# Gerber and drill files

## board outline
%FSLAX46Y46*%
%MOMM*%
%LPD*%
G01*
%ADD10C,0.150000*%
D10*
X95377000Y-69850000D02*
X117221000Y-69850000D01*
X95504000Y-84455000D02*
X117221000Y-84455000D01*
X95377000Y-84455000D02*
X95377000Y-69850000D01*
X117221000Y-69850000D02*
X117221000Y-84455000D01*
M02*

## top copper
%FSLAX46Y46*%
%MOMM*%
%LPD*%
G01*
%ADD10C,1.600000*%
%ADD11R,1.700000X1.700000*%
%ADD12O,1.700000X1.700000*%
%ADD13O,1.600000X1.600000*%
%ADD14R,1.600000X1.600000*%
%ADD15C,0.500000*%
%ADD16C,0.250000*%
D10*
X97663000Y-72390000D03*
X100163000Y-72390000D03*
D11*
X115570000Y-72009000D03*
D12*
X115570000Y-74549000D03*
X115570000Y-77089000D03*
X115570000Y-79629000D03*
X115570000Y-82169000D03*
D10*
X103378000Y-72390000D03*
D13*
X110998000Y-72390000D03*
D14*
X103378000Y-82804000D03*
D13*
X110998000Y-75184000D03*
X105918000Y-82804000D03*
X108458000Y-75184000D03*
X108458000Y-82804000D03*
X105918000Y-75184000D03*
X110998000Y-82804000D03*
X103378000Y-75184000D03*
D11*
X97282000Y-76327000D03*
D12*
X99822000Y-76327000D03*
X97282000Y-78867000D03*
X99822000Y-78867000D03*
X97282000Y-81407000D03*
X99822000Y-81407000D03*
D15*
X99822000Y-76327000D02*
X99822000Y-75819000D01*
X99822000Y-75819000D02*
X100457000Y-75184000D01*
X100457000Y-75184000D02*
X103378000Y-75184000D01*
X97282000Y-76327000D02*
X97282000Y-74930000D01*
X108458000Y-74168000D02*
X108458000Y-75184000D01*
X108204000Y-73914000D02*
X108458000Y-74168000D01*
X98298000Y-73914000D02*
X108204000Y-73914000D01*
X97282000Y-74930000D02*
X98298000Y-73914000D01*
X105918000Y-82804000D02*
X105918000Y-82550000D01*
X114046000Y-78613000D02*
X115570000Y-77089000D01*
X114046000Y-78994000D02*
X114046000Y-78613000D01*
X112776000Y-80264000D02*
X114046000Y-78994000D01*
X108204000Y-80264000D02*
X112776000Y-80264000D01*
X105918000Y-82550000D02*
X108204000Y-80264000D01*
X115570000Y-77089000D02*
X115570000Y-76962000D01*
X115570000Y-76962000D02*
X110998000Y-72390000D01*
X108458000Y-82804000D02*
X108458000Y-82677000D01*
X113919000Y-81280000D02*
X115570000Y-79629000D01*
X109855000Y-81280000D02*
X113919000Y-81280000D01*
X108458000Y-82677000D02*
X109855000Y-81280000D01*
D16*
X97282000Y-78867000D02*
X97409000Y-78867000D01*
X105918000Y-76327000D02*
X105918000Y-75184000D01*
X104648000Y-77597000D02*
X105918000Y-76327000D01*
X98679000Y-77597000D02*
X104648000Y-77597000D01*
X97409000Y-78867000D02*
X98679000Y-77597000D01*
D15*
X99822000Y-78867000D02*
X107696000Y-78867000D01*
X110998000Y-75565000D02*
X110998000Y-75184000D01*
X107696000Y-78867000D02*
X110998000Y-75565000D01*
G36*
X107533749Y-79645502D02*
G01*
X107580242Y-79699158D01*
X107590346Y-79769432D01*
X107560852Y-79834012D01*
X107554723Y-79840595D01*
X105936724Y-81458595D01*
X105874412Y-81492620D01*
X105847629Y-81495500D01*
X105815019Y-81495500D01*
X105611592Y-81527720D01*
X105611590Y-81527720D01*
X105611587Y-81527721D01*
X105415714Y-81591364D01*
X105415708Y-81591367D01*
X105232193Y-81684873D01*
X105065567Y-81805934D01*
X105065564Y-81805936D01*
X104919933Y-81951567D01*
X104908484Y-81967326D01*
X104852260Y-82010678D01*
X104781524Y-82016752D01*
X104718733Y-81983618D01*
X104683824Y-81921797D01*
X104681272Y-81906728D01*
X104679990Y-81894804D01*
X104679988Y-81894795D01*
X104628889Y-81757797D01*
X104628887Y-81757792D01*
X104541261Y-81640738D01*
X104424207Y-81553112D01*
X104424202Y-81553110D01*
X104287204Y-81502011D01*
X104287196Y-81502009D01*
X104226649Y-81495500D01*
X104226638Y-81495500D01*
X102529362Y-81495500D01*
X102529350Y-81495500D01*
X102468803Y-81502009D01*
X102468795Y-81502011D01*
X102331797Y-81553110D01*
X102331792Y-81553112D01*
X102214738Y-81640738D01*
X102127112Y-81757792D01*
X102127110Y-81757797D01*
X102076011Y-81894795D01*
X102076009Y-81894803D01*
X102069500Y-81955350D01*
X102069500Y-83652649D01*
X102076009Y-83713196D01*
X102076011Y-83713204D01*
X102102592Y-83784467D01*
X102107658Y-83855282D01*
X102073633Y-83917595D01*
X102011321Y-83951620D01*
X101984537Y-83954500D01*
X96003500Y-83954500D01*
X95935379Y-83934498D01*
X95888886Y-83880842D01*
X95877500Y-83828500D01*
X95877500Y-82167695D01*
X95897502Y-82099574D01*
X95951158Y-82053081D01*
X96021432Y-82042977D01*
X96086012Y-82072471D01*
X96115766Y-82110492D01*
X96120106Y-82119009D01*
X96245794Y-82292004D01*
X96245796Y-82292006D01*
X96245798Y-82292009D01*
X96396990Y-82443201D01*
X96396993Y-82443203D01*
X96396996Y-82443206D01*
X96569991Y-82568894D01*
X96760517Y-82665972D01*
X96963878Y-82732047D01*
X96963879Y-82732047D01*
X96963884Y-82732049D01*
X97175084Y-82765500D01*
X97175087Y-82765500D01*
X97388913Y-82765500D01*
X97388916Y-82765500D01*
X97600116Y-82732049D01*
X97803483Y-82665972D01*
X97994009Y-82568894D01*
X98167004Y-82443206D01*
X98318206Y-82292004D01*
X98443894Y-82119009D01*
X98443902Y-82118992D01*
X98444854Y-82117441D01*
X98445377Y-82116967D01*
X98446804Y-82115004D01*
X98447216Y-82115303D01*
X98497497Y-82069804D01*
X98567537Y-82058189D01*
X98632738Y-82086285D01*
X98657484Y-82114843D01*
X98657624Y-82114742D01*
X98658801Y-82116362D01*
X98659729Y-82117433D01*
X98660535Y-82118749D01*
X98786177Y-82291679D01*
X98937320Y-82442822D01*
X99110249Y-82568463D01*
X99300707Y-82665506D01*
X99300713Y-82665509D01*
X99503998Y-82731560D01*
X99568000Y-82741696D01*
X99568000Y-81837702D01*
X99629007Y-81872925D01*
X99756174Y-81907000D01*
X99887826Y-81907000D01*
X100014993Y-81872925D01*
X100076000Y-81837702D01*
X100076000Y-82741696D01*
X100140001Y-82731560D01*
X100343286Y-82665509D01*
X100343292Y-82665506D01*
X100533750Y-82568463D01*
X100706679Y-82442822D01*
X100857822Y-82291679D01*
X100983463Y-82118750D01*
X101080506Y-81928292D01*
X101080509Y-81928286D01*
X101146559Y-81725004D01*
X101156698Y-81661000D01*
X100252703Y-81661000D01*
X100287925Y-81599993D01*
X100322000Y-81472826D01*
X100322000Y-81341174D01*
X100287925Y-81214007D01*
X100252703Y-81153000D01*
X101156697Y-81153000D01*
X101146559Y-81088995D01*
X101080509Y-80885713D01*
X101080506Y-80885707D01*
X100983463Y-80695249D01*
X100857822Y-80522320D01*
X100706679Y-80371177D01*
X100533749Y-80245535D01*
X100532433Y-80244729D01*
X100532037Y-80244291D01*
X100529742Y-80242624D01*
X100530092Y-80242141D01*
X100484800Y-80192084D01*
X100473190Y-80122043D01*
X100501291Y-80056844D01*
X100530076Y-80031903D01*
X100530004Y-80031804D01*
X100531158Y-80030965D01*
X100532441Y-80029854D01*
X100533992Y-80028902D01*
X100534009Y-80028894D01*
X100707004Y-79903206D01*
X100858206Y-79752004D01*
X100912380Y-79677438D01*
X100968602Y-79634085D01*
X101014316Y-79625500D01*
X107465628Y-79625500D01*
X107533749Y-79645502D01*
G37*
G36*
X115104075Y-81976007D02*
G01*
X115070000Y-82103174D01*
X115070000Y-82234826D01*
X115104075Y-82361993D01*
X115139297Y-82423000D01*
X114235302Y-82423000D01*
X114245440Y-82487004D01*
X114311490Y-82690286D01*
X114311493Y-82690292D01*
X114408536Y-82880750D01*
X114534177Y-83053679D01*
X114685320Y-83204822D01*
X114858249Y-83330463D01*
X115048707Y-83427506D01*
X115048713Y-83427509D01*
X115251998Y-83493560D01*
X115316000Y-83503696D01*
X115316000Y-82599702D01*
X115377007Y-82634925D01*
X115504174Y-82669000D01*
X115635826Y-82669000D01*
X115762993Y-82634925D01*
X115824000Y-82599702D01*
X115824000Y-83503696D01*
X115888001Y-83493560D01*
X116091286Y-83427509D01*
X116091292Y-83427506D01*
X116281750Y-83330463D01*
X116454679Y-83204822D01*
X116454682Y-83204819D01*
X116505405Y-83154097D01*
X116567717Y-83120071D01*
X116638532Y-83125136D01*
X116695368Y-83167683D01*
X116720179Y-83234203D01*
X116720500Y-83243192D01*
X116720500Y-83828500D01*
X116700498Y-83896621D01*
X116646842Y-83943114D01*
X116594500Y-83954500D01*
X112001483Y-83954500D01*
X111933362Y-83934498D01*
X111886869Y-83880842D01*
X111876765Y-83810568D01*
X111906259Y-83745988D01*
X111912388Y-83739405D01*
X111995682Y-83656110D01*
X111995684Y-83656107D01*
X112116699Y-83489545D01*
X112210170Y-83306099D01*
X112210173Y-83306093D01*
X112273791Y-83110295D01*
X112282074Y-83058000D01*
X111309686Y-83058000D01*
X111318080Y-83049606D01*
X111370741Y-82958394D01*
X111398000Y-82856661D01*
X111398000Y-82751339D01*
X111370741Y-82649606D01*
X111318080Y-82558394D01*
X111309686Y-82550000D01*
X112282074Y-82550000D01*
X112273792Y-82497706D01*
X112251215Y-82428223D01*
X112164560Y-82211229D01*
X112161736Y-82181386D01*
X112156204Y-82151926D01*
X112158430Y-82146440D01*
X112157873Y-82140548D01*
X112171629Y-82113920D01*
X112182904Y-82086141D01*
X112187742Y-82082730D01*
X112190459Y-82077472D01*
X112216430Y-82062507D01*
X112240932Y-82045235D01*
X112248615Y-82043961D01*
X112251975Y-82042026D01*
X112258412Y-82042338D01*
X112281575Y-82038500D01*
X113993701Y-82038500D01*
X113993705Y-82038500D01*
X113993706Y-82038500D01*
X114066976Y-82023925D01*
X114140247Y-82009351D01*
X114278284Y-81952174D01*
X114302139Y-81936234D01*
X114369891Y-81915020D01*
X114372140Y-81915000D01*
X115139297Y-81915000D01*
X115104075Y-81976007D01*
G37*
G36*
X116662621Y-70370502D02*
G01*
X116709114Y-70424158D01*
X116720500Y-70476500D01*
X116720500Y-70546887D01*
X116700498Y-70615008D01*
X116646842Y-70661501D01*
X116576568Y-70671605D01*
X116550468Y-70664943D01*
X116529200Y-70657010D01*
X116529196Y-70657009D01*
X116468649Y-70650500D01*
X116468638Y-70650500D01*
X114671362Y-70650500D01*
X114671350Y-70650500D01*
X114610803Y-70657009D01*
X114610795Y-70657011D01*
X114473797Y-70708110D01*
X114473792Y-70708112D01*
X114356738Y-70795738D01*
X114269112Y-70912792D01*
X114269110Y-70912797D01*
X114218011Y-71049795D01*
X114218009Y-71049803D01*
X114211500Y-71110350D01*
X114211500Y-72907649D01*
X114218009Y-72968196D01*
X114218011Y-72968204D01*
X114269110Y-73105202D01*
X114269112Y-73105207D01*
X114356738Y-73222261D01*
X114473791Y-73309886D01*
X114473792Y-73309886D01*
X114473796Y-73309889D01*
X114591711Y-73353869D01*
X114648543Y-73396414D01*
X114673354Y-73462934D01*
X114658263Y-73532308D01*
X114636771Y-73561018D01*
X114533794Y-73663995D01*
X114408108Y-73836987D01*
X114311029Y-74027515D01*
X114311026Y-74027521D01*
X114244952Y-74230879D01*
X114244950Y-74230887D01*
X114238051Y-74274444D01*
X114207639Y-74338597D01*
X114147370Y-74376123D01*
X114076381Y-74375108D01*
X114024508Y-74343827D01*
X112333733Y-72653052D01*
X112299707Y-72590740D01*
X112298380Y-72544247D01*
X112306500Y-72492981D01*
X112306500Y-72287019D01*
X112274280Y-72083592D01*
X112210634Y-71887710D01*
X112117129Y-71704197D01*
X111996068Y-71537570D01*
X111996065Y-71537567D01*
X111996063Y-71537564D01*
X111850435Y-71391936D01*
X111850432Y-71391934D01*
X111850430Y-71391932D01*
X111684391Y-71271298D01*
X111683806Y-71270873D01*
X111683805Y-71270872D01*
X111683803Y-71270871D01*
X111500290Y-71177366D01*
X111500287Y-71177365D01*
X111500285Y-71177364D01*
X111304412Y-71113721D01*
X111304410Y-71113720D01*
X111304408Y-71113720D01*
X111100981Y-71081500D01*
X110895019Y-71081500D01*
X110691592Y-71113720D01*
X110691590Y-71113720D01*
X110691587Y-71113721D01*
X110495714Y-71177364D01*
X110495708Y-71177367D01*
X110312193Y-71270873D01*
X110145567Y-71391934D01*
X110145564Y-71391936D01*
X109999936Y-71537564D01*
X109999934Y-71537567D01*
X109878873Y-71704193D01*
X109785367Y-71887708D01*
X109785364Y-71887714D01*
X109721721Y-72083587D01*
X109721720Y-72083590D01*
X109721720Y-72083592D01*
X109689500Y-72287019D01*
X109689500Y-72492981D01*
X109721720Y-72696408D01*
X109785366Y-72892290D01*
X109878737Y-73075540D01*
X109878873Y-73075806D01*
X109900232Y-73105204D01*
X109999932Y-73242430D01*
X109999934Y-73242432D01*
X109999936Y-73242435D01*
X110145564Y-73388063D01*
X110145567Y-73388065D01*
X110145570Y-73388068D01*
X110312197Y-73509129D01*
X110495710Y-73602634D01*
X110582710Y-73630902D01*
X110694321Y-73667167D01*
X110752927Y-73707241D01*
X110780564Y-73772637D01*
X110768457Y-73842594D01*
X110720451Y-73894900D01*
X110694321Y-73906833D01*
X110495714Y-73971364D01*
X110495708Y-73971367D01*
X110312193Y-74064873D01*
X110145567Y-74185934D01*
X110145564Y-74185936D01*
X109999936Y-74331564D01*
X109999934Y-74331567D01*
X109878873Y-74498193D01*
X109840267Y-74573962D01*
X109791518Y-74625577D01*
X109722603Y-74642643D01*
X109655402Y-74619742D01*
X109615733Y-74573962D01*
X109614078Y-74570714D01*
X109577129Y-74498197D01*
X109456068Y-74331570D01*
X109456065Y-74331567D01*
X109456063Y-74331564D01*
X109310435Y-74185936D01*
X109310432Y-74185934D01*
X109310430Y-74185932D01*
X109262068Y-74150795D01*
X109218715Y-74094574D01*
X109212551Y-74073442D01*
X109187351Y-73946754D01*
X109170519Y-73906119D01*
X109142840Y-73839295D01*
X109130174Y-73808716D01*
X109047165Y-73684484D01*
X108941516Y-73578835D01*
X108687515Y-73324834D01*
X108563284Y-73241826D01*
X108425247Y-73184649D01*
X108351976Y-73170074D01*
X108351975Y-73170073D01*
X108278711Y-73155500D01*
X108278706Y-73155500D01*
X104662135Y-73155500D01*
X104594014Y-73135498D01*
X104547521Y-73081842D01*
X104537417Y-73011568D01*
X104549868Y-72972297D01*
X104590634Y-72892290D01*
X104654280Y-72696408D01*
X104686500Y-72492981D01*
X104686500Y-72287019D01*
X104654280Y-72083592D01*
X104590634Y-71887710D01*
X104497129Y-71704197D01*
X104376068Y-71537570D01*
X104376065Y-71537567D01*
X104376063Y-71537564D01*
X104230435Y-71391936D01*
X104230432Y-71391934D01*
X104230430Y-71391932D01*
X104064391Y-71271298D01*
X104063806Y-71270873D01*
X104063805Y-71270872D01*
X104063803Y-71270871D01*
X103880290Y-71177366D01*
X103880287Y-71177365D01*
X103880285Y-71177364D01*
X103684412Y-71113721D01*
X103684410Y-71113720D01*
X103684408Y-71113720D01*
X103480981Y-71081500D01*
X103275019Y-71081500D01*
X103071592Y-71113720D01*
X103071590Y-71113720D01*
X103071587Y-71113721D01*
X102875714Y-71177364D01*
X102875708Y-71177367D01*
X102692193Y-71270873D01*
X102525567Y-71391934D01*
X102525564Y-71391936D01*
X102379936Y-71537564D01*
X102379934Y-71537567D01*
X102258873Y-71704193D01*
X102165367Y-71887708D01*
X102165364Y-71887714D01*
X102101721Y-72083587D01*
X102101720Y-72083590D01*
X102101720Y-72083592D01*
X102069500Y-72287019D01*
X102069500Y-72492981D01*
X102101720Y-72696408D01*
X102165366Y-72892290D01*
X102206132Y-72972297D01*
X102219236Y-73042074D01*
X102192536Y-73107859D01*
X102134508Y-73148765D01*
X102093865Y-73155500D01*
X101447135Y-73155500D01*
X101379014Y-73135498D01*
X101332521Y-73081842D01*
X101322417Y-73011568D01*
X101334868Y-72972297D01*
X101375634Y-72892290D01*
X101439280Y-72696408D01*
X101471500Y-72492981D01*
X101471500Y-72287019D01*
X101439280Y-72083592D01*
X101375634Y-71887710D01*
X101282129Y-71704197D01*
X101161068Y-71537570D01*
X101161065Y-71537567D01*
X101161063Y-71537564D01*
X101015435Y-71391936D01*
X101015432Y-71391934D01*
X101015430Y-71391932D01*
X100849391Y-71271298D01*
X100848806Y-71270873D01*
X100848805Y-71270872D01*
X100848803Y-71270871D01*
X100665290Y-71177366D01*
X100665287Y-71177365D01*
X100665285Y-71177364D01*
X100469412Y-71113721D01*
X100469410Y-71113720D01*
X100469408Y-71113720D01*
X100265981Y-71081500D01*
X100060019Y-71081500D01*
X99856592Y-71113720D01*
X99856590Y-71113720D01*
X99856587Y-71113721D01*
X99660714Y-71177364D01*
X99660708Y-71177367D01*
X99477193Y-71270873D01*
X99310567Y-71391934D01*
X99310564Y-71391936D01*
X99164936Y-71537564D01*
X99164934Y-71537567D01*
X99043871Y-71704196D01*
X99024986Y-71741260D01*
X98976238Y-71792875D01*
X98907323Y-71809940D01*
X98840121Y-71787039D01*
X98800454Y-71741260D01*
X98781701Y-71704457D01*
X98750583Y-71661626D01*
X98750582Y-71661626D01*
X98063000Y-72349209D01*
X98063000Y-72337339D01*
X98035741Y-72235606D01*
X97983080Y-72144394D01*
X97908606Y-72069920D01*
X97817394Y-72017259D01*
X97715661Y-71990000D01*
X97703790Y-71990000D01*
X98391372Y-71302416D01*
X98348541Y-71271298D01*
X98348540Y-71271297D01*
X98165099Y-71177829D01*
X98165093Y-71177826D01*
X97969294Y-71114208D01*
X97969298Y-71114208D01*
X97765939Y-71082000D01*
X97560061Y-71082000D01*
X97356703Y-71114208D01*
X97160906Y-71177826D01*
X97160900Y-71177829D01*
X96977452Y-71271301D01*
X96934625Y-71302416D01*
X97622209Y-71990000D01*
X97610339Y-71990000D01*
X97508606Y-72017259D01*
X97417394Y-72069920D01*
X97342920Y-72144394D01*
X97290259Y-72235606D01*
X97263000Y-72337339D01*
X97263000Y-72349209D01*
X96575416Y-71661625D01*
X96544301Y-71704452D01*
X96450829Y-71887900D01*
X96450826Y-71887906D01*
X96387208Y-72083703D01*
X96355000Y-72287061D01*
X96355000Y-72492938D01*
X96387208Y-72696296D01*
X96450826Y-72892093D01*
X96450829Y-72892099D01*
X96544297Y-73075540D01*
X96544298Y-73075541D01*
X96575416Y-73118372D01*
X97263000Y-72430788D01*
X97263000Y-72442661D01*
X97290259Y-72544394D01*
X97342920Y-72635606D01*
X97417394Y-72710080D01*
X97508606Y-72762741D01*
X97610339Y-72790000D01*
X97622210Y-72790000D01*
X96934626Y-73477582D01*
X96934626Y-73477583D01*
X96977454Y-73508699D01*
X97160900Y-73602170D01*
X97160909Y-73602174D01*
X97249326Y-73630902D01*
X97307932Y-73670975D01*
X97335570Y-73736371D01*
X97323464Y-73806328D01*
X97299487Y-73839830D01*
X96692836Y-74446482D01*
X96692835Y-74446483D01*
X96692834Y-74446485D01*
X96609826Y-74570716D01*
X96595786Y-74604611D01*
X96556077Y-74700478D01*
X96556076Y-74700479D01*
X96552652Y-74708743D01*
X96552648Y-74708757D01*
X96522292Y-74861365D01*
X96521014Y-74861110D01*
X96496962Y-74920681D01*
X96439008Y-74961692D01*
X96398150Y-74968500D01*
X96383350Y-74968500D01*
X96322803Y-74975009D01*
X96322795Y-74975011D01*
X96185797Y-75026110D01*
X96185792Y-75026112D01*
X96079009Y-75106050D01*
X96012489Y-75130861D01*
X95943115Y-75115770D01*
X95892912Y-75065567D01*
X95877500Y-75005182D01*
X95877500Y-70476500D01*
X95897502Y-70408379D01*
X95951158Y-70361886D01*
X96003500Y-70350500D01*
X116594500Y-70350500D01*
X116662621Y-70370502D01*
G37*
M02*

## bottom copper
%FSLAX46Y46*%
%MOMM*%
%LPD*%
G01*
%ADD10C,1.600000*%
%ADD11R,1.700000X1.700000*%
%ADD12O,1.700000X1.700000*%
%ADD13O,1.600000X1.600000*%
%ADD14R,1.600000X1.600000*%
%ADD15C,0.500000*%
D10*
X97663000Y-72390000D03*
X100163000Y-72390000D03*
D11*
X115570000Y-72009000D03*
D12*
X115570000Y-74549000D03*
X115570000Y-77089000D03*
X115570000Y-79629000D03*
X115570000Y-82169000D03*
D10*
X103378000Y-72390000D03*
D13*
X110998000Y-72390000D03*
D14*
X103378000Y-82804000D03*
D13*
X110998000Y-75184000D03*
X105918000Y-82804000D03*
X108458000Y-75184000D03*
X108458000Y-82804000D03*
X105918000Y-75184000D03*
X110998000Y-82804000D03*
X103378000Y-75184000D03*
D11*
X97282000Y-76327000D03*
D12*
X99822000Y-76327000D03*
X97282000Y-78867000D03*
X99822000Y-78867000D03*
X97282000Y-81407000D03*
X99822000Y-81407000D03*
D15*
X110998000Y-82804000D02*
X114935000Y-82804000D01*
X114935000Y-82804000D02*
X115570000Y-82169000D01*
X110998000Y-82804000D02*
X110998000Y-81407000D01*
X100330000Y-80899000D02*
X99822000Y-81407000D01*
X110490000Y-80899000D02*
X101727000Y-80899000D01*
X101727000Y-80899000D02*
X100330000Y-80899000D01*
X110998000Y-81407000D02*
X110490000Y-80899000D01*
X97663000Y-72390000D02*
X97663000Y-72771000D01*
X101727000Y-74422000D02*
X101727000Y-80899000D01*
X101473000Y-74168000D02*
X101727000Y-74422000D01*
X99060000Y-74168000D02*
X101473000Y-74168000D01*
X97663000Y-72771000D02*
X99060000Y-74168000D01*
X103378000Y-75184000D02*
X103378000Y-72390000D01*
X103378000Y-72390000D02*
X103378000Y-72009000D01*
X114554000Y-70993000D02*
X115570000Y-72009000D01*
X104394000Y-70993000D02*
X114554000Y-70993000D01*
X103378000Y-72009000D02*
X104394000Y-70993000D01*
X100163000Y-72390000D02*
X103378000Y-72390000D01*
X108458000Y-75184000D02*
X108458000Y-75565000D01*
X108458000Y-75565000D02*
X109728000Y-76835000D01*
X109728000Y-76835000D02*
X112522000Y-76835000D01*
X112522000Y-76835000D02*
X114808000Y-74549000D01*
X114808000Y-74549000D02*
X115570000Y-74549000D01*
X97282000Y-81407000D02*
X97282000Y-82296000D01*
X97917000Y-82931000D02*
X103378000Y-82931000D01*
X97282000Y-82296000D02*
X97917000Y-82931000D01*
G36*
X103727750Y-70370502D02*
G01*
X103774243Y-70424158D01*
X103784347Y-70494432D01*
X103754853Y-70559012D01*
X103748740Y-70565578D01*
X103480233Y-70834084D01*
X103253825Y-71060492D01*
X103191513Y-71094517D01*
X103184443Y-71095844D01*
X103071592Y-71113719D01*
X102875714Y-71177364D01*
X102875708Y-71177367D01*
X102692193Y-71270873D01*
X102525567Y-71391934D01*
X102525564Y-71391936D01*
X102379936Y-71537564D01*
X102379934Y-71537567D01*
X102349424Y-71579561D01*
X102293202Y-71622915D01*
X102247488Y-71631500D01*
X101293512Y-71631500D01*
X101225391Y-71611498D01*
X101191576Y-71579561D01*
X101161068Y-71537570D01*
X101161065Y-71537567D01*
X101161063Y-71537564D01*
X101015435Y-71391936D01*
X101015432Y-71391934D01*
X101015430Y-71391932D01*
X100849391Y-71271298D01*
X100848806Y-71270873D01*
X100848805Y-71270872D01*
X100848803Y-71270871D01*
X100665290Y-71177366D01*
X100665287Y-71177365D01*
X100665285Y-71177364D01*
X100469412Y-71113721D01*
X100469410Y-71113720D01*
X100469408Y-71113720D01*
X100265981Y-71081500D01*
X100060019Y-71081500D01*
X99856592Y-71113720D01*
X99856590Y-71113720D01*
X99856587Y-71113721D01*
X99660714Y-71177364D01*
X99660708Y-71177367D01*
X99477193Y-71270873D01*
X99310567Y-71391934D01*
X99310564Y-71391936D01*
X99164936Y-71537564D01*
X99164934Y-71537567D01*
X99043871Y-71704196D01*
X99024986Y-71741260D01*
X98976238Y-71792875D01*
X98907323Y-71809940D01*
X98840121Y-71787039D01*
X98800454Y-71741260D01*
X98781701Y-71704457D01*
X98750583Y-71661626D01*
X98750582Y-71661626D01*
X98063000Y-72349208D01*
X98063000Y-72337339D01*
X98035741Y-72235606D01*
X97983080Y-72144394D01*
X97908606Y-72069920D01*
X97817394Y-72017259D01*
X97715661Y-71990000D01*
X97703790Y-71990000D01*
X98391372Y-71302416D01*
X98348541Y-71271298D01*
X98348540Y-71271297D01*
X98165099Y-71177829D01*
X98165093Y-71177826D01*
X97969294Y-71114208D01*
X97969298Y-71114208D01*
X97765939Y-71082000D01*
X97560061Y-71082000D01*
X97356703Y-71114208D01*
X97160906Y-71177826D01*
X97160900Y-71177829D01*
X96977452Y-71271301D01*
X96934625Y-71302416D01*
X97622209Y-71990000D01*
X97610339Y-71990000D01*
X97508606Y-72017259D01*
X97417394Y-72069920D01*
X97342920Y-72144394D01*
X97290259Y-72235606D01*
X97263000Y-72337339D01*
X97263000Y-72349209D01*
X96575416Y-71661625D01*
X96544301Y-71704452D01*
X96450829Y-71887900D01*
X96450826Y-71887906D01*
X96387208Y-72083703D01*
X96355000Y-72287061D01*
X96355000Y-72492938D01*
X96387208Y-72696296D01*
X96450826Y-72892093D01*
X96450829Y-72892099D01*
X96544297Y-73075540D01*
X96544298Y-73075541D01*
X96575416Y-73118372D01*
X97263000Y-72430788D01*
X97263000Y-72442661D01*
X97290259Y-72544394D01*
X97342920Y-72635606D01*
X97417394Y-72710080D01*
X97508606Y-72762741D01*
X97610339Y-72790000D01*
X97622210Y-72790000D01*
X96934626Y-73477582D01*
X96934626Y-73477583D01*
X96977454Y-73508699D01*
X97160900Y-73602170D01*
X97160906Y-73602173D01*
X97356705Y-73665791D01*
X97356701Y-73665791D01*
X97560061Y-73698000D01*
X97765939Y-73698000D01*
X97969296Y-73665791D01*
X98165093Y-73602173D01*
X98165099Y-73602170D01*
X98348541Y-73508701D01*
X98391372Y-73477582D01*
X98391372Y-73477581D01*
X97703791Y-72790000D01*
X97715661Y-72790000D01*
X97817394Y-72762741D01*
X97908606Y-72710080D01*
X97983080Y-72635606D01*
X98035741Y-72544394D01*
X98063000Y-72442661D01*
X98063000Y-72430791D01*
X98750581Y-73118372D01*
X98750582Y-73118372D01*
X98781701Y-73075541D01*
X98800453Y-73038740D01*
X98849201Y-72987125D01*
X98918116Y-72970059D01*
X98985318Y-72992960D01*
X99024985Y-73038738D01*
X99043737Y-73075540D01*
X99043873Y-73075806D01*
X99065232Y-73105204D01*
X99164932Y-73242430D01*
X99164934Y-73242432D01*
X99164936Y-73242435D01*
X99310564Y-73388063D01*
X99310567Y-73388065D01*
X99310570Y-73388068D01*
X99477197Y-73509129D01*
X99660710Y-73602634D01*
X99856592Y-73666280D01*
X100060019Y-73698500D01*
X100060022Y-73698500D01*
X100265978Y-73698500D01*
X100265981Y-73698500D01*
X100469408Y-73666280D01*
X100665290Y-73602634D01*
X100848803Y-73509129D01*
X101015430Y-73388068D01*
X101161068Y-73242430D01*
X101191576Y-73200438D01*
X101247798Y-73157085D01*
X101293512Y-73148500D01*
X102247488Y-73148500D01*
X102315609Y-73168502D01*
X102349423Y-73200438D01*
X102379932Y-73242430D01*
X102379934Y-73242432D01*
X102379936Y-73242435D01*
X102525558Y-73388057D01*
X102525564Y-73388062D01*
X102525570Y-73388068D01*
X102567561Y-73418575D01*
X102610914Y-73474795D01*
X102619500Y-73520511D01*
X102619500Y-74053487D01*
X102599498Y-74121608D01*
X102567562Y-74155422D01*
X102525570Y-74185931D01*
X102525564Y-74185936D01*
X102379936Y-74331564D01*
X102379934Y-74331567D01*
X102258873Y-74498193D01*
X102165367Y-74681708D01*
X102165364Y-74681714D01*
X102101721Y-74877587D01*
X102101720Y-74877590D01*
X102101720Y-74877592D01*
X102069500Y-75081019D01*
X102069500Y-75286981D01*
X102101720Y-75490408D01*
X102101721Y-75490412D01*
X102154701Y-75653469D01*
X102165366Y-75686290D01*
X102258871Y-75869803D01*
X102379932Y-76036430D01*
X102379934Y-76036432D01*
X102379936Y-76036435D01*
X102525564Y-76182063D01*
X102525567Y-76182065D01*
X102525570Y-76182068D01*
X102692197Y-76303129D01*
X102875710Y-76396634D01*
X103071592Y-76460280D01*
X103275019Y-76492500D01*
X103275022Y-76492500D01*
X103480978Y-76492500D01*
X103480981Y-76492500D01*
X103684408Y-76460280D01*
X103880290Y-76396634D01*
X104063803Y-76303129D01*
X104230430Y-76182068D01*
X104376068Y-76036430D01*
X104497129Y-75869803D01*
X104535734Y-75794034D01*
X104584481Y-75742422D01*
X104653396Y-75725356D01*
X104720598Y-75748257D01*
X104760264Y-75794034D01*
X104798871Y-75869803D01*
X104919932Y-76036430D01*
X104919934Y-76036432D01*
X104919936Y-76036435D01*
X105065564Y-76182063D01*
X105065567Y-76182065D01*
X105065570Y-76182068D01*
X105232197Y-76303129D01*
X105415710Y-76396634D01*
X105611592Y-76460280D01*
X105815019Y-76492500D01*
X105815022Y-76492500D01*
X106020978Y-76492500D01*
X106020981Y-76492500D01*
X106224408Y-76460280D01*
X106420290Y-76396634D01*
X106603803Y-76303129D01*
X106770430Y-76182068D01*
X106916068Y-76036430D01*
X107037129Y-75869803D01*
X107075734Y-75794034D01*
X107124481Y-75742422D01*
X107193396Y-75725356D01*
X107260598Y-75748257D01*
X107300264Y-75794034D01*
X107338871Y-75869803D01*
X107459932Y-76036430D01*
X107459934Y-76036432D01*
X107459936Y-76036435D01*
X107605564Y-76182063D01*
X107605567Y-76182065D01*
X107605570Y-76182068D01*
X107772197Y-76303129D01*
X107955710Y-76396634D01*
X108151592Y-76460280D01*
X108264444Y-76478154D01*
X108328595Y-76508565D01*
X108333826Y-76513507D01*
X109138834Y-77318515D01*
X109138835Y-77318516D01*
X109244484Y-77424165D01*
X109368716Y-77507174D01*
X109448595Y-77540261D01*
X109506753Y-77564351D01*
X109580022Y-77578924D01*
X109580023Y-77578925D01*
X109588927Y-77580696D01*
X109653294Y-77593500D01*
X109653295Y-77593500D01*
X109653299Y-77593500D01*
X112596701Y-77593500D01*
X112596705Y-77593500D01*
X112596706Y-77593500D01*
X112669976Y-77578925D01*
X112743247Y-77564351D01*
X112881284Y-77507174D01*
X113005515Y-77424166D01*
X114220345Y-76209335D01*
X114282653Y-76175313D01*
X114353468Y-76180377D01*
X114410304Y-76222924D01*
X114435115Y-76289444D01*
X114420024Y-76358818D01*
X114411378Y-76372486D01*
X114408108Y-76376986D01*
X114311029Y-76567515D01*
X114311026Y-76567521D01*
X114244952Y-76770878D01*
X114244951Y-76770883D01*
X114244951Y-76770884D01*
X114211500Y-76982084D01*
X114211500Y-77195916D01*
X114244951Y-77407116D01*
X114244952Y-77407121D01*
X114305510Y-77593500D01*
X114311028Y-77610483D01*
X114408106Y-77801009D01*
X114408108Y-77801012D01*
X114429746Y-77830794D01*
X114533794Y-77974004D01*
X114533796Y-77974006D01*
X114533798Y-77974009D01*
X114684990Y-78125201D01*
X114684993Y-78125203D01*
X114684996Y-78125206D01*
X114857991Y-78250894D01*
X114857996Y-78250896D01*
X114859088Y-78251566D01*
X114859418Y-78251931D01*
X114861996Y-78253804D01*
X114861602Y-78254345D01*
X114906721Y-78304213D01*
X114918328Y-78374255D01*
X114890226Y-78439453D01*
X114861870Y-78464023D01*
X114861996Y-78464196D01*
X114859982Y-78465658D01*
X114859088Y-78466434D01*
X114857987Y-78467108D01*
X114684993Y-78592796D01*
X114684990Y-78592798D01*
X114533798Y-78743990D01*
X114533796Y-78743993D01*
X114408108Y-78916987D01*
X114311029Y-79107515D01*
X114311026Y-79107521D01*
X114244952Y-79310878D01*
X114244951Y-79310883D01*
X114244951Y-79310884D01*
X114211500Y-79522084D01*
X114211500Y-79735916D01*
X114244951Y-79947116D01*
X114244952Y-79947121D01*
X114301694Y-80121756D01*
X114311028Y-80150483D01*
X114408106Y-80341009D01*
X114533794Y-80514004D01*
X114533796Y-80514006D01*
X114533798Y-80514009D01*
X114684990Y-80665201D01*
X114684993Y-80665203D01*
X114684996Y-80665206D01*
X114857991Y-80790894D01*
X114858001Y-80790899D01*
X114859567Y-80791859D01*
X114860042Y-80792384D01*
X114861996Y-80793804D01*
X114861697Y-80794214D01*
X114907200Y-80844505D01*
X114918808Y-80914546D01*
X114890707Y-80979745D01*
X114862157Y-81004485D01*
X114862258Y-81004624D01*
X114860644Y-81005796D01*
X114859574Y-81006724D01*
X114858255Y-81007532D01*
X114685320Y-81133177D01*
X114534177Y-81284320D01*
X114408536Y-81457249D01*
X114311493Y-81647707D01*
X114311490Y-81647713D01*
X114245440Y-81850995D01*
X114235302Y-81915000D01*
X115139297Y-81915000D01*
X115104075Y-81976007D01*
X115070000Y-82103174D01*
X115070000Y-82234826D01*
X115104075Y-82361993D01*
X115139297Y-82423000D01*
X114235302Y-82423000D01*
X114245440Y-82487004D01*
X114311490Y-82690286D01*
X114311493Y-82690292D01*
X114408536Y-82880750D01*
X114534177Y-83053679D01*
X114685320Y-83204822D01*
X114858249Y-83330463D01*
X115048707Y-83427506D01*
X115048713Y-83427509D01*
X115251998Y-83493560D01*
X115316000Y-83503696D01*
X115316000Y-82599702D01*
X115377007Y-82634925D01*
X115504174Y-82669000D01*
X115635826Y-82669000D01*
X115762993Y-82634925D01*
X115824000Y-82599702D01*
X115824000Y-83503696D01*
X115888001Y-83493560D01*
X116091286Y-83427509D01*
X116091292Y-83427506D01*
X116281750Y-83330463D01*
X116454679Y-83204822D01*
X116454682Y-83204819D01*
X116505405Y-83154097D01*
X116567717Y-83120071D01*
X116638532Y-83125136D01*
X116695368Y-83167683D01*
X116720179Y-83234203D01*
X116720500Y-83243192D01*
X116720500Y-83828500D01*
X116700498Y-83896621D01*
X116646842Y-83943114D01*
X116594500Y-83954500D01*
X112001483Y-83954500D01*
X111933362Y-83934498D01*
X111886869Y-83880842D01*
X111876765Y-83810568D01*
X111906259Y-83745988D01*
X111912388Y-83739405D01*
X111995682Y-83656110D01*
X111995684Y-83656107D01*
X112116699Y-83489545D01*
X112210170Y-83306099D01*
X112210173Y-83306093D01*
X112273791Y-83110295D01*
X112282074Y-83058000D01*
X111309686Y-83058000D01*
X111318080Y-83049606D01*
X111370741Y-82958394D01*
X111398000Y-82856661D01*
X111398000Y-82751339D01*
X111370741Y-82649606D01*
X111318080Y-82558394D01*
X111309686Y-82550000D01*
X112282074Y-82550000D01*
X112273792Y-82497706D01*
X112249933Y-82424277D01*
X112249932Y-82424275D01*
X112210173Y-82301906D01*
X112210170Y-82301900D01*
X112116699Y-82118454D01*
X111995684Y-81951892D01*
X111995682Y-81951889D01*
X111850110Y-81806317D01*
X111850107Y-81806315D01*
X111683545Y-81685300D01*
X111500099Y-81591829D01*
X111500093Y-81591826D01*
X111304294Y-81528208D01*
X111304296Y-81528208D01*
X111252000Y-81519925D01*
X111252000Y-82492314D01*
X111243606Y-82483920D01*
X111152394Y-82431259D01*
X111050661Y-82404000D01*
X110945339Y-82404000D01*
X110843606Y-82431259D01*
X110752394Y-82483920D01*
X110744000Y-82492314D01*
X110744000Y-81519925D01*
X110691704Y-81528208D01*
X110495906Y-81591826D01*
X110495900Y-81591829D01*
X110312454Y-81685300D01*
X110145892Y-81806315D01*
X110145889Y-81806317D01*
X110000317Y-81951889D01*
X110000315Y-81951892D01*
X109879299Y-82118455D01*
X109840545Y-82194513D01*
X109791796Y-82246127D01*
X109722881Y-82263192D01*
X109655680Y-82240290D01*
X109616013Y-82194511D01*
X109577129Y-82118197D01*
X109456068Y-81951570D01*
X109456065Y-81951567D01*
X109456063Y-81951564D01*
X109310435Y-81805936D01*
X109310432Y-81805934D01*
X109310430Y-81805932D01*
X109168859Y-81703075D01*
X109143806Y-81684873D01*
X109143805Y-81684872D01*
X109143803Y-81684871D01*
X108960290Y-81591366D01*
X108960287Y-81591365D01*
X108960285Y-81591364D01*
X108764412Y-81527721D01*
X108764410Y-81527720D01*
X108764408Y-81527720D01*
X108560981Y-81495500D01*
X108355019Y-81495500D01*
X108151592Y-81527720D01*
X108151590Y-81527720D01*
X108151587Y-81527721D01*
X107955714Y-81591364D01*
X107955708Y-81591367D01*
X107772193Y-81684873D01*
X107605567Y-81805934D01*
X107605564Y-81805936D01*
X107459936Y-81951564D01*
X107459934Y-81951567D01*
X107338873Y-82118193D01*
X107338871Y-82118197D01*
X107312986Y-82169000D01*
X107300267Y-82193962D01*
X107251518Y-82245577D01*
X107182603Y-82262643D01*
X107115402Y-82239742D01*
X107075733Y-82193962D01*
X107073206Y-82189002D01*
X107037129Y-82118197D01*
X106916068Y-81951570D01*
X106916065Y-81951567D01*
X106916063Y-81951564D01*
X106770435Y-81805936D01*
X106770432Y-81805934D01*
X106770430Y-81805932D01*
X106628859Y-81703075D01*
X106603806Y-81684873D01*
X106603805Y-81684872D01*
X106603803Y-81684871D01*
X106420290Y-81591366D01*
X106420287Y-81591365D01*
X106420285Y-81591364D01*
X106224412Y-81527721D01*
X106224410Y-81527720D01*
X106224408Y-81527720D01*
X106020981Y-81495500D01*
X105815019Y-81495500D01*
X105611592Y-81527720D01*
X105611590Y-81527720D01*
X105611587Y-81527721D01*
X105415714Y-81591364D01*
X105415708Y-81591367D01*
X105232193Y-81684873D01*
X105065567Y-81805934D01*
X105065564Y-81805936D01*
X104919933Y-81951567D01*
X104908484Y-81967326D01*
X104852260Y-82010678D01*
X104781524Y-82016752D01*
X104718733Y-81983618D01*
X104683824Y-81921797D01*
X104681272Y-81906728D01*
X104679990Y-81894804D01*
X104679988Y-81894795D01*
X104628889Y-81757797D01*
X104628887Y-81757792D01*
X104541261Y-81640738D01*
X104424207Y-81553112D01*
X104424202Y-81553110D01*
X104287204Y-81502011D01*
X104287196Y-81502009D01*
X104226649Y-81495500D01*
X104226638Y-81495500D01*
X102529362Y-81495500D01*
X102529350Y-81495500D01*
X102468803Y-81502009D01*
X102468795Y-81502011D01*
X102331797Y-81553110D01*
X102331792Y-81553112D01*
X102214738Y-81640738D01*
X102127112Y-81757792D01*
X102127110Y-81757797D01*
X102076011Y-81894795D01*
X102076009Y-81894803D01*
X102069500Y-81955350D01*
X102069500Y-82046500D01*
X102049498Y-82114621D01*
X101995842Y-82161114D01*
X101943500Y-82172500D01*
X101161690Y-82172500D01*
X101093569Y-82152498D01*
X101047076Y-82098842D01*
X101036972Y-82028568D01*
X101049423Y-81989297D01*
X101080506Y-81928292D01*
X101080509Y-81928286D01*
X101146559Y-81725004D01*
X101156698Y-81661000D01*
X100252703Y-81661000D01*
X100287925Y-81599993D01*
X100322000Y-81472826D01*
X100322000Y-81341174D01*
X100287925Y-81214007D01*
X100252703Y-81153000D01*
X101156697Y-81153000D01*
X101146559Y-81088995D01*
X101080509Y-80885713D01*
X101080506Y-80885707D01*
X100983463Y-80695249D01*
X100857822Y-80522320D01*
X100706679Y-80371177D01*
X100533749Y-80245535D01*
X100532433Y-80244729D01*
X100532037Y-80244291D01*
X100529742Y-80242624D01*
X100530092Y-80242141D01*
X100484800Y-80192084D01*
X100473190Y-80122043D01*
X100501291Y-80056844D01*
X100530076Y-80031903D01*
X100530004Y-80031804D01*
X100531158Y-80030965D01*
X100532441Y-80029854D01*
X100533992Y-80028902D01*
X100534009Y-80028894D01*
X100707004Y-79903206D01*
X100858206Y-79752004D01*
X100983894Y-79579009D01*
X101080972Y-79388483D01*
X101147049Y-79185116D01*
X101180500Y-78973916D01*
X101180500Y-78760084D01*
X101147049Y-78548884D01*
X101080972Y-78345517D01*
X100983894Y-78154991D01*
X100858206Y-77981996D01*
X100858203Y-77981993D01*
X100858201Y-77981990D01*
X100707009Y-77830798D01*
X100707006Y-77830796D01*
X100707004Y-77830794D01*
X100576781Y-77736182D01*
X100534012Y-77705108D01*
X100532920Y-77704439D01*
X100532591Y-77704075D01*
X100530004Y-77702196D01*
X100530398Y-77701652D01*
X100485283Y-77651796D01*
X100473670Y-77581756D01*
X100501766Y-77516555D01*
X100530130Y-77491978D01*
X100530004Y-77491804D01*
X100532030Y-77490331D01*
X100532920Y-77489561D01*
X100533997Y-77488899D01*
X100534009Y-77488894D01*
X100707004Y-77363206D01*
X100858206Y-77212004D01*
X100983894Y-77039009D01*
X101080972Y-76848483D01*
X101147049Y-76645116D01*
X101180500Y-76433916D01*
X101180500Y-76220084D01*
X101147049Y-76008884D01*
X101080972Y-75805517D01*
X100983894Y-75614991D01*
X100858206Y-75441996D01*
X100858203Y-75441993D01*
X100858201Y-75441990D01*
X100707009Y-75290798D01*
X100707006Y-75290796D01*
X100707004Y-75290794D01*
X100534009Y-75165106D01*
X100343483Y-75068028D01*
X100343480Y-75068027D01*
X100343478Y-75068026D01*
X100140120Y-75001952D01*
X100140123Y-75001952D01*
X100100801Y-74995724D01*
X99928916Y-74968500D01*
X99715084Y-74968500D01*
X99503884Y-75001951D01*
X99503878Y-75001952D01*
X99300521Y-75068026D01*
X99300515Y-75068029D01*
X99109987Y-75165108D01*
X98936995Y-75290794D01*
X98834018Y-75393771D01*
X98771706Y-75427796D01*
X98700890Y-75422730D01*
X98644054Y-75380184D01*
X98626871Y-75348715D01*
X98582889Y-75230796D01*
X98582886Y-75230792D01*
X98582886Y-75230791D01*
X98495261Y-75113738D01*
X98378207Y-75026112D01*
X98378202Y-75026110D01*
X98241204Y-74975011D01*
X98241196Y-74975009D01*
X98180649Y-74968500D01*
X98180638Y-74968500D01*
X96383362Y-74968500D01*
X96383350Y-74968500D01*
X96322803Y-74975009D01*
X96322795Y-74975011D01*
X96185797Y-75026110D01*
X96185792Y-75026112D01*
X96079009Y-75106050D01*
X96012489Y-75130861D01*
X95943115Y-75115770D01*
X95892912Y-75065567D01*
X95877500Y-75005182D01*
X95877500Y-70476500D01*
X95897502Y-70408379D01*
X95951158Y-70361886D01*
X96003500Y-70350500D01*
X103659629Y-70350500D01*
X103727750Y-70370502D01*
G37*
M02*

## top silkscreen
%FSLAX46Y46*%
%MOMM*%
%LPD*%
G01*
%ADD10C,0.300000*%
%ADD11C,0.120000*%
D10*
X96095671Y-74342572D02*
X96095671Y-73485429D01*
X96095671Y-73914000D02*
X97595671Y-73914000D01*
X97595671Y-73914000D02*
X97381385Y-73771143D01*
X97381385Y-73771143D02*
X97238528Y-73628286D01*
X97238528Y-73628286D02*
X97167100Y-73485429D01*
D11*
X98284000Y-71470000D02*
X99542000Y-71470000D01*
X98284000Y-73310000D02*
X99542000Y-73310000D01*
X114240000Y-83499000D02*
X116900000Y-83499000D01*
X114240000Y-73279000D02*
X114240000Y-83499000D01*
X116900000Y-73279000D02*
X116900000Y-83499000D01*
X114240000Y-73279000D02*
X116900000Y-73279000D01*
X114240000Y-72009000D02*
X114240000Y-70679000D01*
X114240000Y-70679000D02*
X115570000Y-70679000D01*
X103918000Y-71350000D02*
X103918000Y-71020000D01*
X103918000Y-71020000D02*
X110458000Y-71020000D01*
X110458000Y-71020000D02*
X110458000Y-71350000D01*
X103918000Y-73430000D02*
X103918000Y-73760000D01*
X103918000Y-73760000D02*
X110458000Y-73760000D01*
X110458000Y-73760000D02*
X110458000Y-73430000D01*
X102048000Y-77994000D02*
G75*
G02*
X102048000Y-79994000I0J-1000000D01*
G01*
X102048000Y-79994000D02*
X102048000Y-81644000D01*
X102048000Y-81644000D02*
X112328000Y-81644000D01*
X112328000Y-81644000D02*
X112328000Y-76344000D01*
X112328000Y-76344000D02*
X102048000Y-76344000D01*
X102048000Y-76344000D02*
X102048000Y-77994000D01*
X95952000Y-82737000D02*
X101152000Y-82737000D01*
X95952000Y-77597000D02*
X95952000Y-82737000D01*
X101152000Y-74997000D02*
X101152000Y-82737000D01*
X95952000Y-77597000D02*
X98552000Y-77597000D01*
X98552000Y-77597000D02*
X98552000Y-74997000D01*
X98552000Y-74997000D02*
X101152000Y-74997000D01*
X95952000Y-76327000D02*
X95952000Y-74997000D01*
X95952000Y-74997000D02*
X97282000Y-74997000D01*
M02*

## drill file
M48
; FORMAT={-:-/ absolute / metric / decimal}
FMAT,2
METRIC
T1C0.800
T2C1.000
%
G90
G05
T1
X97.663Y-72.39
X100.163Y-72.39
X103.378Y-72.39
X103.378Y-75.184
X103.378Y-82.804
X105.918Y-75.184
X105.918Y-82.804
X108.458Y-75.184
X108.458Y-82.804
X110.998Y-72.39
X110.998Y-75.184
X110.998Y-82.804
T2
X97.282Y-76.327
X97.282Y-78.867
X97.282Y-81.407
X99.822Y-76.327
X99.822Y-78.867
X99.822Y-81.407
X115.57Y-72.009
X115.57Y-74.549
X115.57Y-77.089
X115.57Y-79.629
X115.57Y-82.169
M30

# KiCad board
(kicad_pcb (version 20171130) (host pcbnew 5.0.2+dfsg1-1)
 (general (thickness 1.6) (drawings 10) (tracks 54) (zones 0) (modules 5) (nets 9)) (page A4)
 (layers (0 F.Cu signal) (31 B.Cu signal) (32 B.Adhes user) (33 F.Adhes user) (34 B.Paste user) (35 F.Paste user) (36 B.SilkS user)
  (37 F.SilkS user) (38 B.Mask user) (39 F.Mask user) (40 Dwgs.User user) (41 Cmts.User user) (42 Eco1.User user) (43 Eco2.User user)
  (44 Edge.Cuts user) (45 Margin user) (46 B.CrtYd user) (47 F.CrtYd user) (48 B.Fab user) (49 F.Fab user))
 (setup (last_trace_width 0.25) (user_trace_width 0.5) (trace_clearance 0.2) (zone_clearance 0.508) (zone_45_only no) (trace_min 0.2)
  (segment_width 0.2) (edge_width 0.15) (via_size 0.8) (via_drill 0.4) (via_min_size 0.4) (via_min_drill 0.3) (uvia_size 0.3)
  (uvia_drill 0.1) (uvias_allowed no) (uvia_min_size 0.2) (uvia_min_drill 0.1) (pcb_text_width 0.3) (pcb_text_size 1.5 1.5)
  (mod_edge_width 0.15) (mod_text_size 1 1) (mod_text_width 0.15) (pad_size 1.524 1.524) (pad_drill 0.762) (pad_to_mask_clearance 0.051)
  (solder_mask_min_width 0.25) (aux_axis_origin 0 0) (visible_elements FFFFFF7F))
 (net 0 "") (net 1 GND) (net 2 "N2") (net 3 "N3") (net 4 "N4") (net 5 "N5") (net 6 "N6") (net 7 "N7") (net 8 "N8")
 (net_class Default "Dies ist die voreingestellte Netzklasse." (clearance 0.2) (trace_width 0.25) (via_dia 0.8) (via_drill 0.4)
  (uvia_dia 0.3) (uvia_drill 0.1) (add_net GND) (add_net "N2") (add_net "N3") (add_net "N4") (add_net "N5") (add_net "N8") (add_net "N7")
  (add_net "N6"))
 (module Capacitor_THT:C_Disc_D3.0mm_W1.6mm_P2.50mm (layer F.Cu) (at 97.663 72.39)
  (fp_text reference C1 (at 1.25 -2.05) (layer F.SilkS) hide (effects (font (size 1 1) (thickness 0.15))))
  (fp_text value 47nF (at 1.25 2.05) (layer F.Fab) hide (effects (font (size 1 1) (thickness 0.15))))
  (fp_line (start 0.621 -0.92) (end 1.879 -0.92) (layer F.SilkS) (width 0.12))
  (fp_line (start 0.621 0.92) (end 1.879 0.92) (layer F.SilkS) (width 0.12))
  (pad 1 thru_hole circle (at 0 0) (size 1.6 1.6) (drill 0.8) (layers *.Cu *.Mask) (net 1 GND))
  (pad 2 thru_hole circle (at 2.5 0) (size 1.6 1.6) (drill 0.8) (layers *.Cu *.Mask) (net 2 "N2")))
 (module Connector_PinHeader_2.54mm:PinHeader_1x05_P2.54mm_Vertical (layer F.Cu) (at 115.57 72.009)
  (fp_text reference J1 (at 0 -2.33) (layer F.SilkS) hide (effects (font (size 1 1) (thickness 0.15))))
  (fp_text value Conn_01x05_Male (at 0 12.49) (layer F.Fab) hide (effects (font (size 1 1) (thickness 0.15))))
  (fp_line (start -1.33 11.49) (end 1.33 11.49) (layer F.SilkS) (width 0.12))
  (fp_line (start -1.33 1.27) (end -1.33 11.49) (layer F.SilkS) (width 0.12))
  (fp_line (start 1.33 1.27) (end 1.33 11.49) (layer F.SilkS) (width 0.12))
  (fp_line (start -1.33 1.27) (end 1.33 1.27) (layer F.SilkS) (width 0.12))
  (fp_line (start -1.33 0) (end -1.33 -1.33) (layer F.SilkS) (width 0.12))
  (fp_line (start -1.33 -1.33) (end 0 -1.33) (layer F.SilkS) (width 0.12))
  (pad 1 thru_hole rect (at 0 0) (size 1.7 1.7) (drill 1) (layers *.Cu *.Mask) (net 2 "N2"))
  (pad 2 thru_hole oval (at 0 2.54) (size 1.7 1.7) (drill 1) (layers *.Cu *.Mask) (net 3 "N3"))
  (pad 3 thru_hole oval (at 0 5.08) (size 1.7 1.7) (drill 1) (layers *.Cu *.Mask) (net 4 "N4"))
  (pad 4 thru_hole oval (at 0 7.62) (size 1.7 1.7) (drill 1) (layers *.Cu *.Mask) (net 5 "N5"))
  (pad 5 thru_hole oval (at 0 10.16) (size 1.7 1.7) (drill 1) (layers *.Cu *.Mask) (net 1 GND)))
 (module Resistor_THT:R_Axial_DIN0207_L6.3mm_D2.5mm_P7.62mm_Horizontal (layer F.Cu) (at 103.378 72.39)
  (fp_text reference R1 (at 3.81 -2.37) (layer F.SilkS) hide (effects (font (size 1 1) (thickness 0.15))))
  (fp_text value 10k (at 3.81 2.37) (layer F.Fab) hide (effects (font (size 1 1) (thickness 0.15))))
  (fp_line (start 0.54 -1.04) (end 0.54 -1.37) (layer F.SilkS) (width 0.12))
  (fp_line (start 0.54 -1.37) (end 7.08 -1.37) (layer F.SilkS) (width 0.12))
  (fp_line (start 7.08 -1.37) (end 7.08 -1.04) (layer F.SilkS) (width 0.12))
  (fp_line (start 0.54 1.04) (end 0.54 1.37) (layer F.SilkS) (width 0.12))
  (fp_line (start 0.54 1.37) (end 7.08 1.37) (layer F.SilkS) (width 0.12))
  (fp_line (start 7.08 1.37) (end 7.08 1.04) (layer F.SilkS) (width 0.12))
  (pad 1 thru_hole circle (at 0 0) (size 1.6 1.6) (drill 0.8) (layers *.Cu *.Mask) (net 2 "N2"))
  (pad 2 thru_hole oval (at 7.62 0) (size 1.6 1.6) (drill 0.8) (layers *.Cu *.Mask) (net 4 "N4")))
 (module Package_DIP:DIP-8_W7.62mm (layer F.Cu) (at 103.378 82.804 90)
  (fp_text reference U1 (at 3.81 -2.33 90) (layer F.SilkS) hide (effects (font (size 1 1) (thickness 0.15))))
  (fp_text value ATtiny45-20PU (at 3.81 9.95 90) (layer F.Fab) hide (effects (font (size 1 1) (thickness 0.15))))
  (fp_arc (start 3.81 -1.33) (end 2.81 -1.33) (angle -180) (layer F.SilkS) (width 0.12))
  (fp_line (start 2.81 -1.33) (end 1.16 -1.33) (layer F.SilkS) (width 0.12))
  (fp_line (start 1.16 -1.33) (end 1.16 8.95) (layer F.SilkS) (width 0.12))
  (fp_line (start 1.16 8.95) (end 6.46 8.95) (layer F.SilkS) (width 0.12))
  (fp_line (start 6.46 8.95) (end 6.46 -1.33) (layer F.SilkS) (width 0.12))
  (fp_line (start 6.46 -1.33) (end 4.81 -1.33) (layer F.SilkS) (width 0.12))
  (pad 1 thru_hole rect (at 0 0 90) (size 1.6 1.6) (drill 0.8) (layers *.Cu *.Mask) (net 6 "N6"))
  (pad 5 thru_hole oval (at 7.62 7.62 90) (size 1.6 1.6) (drill 0.8) (layers *.Cu *.Mask) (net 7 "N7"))
  (pad 2 thru_hole oval (at 0 2.54 90) (size 1.6 1.6) (drill 0.8) (layers *.Cu *.Mask) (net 4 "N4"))
  (pad 6 thru_hole oval (at 7.62 5.08 90) (size 1.6 1.6) (drill 0.8) (layers *.Cu *.Mask) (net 3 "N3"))
  (pad 3 thru_hole oval (at 0 5.08 90) (size 1.6 1.6) (drill 0.8) (layers *.Cu *.Mask) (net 5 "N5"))
  (pad 7 thru_hole oval (at 7.62 2.54 90) (size 1.6 1.6) (drill 0.8) (layers *.Cu *.Mask) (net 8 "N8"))
  (pad 4 thru_hole oval (at 0 7.62 90) (size 1.6 1.6) (drill 0.8) (layers *.Cu *.Mask) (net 1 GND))
  (pad 8 thru_hole oval (at 7.62 0 90) (size 1.6 1.6) (drill 0.8) (layers *.Cu *.Mask) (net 2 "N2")))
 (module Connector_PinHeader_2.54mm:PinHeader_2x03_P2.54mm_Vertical (layer F.Cu) (at 97.282 76.327)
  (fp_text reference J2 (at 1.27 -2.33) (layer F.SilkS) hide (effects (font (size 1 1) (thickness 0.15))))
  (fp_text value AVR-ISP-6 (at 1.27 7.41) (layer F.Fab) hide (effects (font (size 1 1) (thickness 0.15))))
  (fp_line (start -1.33 6.41) (end 3.87 6.41) (layer F.SilkS) (width 0.12))
  (fp_line (start -1.33 1.27) (end -1.33 6.41) (layer F.SilkS) (width 0.12))
  (fp_line (start 3.87 -1.33) (end 3.87 6.41) (layer F.SilkS) (width 0.12))
  (fp_line (start -1.33 1.27) (end 1.27 1.27) (layer F.SilkS) (width 0.12))
  (fp_line (start 1.27 1.27) (end 1.27 -1.33) (layer F.SilkS) (width 0.12))
  (fp_line (start 1.27 -1.33) (end 3.87 -1.33) (layer F.SilkS) (width 0.12))
  (fp_line (start -1.33 0) (end -1.33 -1.33) (layer F.SilkS) (width 0.12))
  (fp_line (start -1.33 -1.33) (end 0 -1.33) (layer F.SilkS) (width 0.12))
  (pad 1 thru_hole rect (at 0 0) (size 1.7 1.7) (drill 1) (layers *.Cu *.Mask) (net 3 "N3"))
  (pad 2 thru_hole oval (at 2.54 0) (size 1.7 1.7) (drill 1) (layers *.Cu *.Mask) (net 2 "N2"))
  (pad 3 thru_hole oval (at 0 2.54) (size 1.7 1.7) (drill 1) (layers *.Cu *.Mask) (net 8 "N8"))
  (pad 4 thru_hole oval (at 2.54 2.54) (size 1.7 1.7) (drill 1) (layers *.Cu *.Mask) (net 7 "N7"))
  (pad 5 thru_hole oval (at 0 5.08) (size 1.7 1.7) (drill 1) (layers *.Cu *.Mask) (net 6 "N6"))
  (pad 6 thru_hole oval (at 2.54 5.08) (size 1.7 1.7) (drill 1) (layers *.Cu *.Mask) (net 1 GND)))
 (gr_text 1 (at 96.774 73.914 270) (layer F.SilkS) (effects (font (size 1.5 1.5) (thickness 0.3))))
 (gr_line (start 95.377 69.85) (end 117.221 69.85) (angle 90) (layer Edge.Cuts) (width 0.15))
 (gr_line (start 95.504 84.455) (end 117.221 84.455) (angle 90) (layer Edge.Cuts) (width 0.15))
 (gr_line (start 95.377 84.455) (end 95.377 69.85) (angle 90) (layer Edge.Cuts) (width 0.15))
 (gr_line (start 117.221 69.85) (end 117.221 84.455) (angle 90) (layer Edge.Cuts) (width 0.15))
 (segment (start 110.998 82.804) (end 114.935 82.804) (width 0.5) (layer B.Cu) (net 1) (status C00000))
 (segment (start 114.935 82.804) (end 115.57 82.169) (width 0.5) (layer B.Cu) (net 1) (status C00000))
 (segment (start 110.998 82.804) (end 110.998 81.407) (width 0.5) (layer B.Cu) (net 1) (status 400000))
 (segment (start 100.33 80.899) (end 99.822 81.407) (width 0.5) (layer B.Cu) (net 1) (status C00000))
 (segment (start 110.49 80.899) (end 101.727 80.899) (width 0.5) (layer B.Cu) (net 1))
 (segment (start 101.727 80.899) (end 100.33 80.899) (width 0.5) (layer B.Cu) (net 1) (status 800000))
 (segment (start 110.998 81.407) (end 110.49 80.899) (width 0.5) (layer B.Cu) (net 1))
 (segment (start 97.663 72.39) (end 97.663 72.771) (width 0.5) (layer B.Cu) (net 1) (status C00000))
 (segment (start 101.727 74.422) (end 101.727 80.899) (width 0.5) (layer B.Cu) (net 1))
 (segment (start 101.473 74.168) (end 101.727 74.422) (width 0.5) (layer B.Cu) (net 1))
 (segment (start 99.06 74.168) (end 101.473 74.168) (width 0.5) (layer B.Cu) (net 1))
 (segment (start 97.663 72.771) (end 99.06 74.168) (width 0.5) (layer B.Cu) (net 1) (status 400000))
 (segment (start 103.378 75.184) (end 103.378 72.39) (width 0.5) (layer B.Cu) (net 2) (status C00000))
 (segment (start 103.378 72.39) (end 103.378 72.009) (width 0.5) (layer B.Cu) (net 2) (status C00000))
 (segment (start 114.554 70.993) (end 115.57 72.009) (width 0.5) (layer B.Cu) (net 2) (status 800000))
 (segment (start 104.394 70.993) (end 114.554 70.993) (width 0.5) (layer B.Cu) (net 2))
 (segment (start 103.378 72.009) (end 104.394 70.993) (width 0.5) (layer B.Cu) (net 2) (status 400000))
 (segment (start 100.163 72.39) (end 103.378 72.39) (width 0.5) (layer B.Cu) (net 2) (status C00000))
 (segment (start 99.822 76.327) (end 99.822 75.819) (width 0.5) (layer F.Cu) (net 2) (status C00000))
 (segment (start 99.822 75.819) (end 100.457 75.184) (width 0.5) (layer F.Cu) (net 2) (status 400000))
 (segment (start 100.457 75.184) (end 103.378 75.184) (width 0.5) (layer F.Cu) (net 2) (status 800000))
 (segment (start 108.458 75.184) (end 108.458 75.565) (width 0.5) (layer B.Cu) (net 3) (status C00000))
 (segment (start 108.458 75.565) (end 109.728 76.835) (width 0.5) (layer B.Cu) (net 3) (status 400000))
 (segment (start 109.728 76.835) (end 112.522 76.835) (width 0.5) (layer B.Cu) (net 3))
 (segment (start 112.522 76.835) (end 114.808 74.549) (width 0.5) (layer B.Cu) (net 3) (status 800000))
 (segment (start 114.808 74.549) (end 115.57 74.549) (width 0.5) (layer B.Cu) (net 3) (status C00000))
 (segment (start 97.282 76.327) (end 97.282 74.93) (width 0.5) (layer F.Cu) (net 3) (status 400000))
 (segment (start 108.458 74.168) (end 108.458 75.184) (width 0.5) (layer F.Cu) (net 3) (status 800000))
 (segment (start 108.204 73.914) (end 108.458 74.168) (width 0.5) (layer F.Cu) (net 3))
 (segment (start 98.298 73.914) (end 108.204 73.914) (width 0.5) (layer F.Cu) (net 3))
 (segment (start 97.282 74.93) (end 98.298 73.914) (width 0.5) (layer F.Cu) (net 3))
 (segment (start 105.918 82.804) (end 105.918 82.55) (width 0.5) (layer F.Cu) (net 4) (status C00000))
 (segment (start 114.046 78.613) (end 115.57 77.089) (width 0.5) (layer F.Cu) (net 4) (status 800000))
 (segment (start 114.046 78.994) (end 114.046 78.613) (width 0.5) (layer F.Cu) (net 4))
 (segment (start 112.776 80.264) (end 114.046 78.994) (width 0.5) (layer F.Cu) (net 4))
 (segment (start 108.204 80.264) (end 112.776 80.264) (width 0.5) (layer F.Cu) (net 4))
 (segment (start 105.918 82.55) (end 108.204 80.264) (width 0.5) (layer F.Cu) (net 4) (status 400000))
 (segment (start 115.57 77.089) (end 115.57 76.962) (width 0.5) (layer F.Cu) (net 4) (status C00000))
 (segment (start 115.57 76.962) (end 110.998 72.39) (width 0.5) (layer F.Cu) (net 4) (status C00000))
 (segment (start 108.458 82.804) (end 108.458 82.677) (width 0.5) (layer F.Cu) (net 5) (status C00000))
 (segment (start 113.919 81.28) (end 115.57 79.629) (width 0.5) (layer F.Cu) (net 5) (status 800000))
 (segment (start 109.855 81.28) (end 113.919 81.28) (width 0.5) (layer F.Cu) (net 5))
 (segment (start 108.458 82.677) (end 109.855 81.28) (width 0.5) (layer F.Cu) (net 5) (status 400000))
 (segment (start 97.282 78.867) (end 97.409 78.867) (width 0.25) (layer F.Cu) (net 8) (status C00000))
 (segment (start 105.918 76.327) (end 105.918 75.184) (width 0.25) (layer F.Cu) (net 8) (status 800000))
 (segment (start 104.648 77.597) (end 105.918 76.327) (width 0.25) (layer F.Cu) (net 8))
 (segment (start 98.679 77.597) (end 104.648 77.597) (width 0.25) (layer F.Cu) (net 8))
 (segment (start 97.409 78.867) (end 98.679 77.597) (width 0.25) (layer F.Cu) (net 8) (status 400000))
 (segment (start 99.822 78.867) (end 107.696 78.867) (width 0.5) (layer F.Cu) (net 7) (status 400000))
 (segment (start 110.998 75.565) (end 110.998 75.184) (width 0.5) (layer F.Cu) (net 7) (status C00000))
 (segment (start 107.696 78.867) (end 110.998 75.565) (width 0.5) (layer F.Cu) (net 7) (status 800000))
 (segment (start 97.282 81.407) (end 97.282 82.296) (width 0.5) (layer B.Cu) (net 6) (status 400000))
 (segment (start 97.917 82.931) (end 103.378 82.931) (width 0.5) (layer B.Cu) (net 6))
 (segment (start 97.282 82.296) (end 97.917 82.931) (width 0.5) (layer B.Cu) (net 6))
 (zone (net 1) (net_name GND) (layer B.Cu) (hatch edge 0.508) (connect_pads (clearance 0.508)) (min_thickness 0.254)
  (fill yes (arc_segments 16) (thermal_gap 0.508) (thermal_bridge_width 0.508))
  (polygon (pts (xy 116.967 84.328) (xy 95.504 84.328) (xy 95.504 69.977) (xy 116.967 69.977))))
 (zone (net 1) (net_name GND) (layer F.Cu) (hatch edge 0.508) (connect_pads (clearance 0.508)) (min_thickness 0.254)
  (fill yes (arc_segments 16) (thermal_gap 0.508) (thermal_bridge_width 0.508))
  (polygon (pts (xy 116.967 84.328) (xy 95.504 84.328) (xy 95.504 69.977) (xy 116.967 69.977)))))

